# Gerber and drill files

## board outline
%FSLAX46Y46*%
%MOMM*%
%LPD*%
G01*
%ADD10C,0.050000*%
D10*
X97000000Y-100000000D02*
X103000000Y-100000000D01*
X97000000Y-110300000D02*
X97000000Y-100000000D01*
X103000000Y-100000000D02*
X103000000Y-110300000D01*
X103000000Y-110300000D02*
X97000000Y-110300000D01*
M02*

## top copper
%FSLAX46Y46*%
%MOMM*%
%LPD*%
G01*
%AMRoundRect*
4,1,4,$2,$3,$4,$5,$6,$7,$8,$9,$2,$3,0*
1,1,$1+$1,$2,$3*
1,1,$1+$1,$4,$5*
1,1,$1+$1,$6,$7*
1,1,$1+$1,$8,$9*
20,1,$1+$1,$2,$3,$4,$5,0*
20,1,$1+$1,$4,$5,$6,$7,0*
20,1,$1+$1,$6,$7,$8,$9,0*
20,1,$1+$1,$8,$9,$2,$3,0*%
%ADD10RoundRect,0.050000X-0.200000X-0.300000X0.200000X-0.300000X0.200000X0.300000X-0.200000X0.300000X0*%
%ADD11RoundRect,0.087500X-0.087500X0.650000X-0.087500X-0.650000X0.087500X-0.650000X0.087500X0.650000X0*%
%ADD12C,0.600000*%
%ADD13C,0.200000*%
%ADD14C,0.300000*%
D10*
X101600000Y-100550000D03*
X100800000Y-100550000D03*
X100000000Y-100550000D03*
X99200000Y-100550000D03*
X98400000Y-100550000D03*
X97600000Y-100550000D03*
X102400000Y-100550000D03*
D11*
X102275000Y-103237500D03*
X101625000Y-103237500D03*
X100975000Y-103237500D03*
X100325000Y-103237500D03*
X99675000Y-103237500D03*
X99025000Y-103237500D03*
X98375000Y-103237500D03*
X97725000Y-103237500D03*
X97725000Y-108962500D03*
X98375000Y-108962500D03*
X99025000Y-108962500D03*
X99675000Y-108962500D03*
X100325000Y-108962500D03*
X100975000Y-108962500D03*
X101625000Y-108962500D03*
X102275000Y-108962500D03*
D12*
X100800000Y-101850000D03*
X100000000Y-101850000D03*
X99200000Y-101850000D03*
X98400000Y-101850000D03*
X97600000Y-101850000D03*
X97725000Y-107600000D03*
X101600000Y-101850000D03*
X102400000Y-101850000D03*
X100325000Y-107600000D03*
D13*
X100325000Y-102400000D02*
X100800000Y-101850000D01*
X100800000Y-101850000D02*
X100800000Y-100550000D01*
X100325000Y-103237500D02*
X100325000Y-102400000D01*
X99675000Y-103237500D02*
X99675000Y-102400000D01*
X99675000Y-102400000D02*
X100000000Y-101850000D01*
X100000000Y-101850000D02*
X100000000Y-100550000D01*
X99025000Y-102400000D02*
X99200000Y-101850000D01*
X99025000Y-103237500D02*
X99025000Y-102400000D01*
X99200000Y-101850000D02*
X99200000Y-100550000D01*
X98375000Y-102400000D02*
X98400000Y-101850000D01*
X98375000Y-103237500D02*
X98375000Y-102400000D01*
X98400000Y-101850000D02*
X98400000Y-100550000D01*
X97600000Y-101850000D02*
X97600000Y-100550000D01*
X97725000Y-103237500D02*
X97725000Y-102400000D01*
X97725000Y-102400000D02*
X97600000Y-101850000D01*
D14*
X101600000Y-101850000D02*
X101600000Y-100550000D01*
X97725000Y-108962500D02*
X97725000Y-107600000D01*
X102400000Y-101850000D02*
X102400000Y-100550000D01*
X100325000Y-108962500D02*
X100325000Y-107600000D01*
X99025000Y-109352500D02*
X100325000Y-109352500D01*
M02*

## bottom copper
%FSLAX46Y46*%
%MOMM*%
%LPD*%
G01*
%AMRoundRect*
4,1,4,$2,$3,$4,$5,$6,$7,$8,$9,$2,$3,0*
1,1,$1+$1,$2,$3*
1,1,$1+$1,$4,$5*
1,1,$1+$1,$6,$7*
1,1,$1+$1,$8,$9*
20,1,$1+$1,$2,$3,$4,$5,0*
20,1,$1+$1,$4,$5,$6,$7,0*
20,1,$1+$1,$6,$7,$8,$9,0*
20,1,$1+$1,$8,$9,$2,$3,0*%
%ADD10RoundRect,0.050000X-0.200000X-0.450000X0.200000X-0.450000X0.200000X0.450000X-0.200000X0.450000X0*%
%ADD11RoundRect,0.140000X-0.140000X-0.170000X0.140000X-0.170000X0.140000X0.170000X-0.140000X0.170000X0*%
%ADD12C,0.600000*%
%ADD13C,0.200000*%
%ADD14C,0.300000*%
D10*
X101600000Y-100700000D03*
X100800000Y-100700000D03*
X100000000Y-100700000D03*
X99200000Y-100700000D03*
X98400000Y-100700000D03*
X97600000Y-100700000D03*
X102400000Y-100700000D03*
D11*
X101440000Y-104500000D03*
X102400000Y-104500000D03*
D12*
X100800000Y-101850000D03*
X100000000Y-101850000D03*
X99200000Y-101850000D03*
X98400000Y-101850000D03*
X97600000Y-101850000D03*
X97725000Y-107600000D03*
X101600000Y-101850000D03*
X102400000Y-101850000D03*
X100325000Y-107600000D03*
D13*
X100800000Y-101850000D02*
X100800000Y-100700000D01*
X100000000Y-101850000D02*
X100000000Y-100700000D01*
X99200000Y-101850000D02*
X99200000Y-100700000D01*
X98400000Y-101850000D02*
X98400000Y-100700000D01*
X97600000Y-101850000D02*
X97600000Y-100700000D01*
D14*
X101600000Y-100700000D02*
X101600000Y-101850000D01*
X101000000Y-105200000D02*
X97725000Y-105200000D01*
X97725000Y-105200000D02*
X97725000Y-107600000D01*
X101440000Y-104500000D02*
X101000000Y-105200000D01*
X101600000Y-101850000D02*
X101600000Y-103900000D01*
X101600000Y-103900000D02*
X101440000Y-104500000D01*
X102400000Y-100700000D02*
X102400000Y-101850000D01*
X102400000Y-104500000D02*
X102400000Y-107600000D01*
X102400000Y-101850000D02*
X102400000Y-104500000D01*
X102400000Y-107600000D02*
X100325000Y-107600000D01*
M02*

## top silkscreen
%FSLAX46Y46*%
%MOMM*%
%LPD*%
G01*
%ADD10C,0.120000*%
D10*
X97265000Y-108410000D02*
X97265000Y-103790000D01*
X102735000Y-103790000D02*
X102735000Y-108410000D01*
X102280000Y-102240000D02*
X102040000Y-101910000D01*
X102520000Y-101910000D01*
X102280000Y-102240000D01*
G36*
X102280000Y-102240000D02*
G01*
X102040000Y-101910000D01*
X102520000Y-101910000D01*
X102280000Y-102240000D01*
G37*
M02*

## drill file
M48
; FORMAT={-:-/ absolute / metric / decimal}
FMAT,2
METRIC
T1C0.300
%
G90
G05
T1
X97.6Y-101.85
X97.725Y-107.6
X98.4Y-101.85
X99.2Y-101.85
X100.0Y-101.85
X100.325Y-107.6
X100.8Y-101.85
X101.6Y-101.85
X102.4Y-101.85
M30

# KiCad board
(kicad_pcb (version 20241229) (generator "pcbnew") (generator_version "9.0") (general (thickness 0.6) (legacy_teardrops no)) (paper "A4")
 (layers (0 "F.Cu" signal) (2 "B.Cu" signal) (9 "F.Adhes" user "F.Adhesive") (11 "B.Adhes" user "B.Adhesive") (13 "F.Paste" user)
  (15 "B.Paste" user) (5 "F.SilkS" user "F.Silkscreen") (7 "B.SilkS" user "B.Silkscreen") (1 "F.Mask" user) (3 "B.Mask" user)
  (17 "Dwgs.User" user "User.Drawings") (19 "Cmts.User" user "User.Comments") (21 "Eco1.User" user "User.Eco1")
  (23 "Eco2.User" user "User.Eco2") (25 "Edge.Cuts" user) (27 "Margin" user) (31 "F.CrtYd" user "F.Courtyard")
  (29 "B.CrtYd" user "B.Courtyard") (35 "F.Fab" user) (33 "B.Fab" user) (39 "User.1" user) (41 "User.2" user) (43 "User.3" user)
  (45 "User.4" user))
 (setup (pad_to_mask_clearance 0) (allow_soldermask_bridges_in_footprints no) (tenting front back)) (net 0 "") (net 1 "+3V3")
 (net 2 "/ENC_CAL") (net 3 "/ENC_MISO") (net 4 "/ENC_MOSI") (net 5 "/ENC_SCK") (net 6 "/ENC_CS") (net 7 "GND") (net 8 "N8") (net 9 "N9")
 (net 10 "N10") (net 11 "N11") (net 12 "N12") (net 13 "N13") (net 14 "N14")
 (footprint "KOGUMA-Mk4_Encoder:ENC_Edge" (layer "F.Cu") (at 100 100)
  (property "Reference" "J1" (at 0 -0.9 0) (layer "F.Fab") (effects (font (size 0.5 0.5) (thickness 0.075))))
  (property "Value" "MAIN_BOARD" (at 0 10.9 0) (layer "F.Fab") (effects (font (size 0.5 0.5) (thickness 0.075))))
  (pad "1" smd roundrect (at 1.6 0.55) (size 0.5 0.7) (layers "F.Cu" "F.Mask" "F.Paste") (roundrect_rratio 0.1) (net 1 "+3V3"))
  (pad "1" smd roundrect (at 1.6 0.7) (size 0.5 1) (layers "B.Cu" "B.Mask" "B.Paste") (roundrect_rratio 0.1) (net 1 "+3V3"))
  (pad "2" smd roundrect (at 0.8 0.55) (size 0.5 0.7) (layers "F.Cu" "F.Mask" "F.Paste") (roundrect_rratio 0.1) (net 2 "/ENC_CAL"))
  (pad "2" smd roundrect (at 0.8 0.7) (size 0.5 1) (layers "B.Cu" "B.Mask" "B.Paste") (roundrect_rratio 0.1) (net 2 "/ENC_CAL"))
  (pad "3" smd roundrect (at 0 0.55) (size 0.5 0.7) (layers "F.Cu" "F.Mask" "F.Paste") (roundrect_rratio 0.1) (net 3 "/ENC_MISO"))
  (pad "3" smd roundrect (at 0 0.7) (size 0.5 1) (layers "B.Cu" "B.Mask" "B.Paste") (roundrect_rratio 0.1) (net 3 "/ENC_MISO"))
  (pad "4" smd roundrect (at -0.8 0.55) (size 0.5 0.7) (layers "F.Cu" "F.Mask" "F.Paste") (roundrect_rratio 0.1) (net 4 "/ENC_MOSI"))
  (pad "4" smd roundrect (at -0.8 0.7) (size 0.5 1) (layers "B.Cu" "B.Mask" "B.Paste") (roundrect_rratio 0.1) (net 4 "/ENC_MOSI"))
  (pad "5" smd roundrect (at -1.6 0.55) (size 0.5 0.7) (layers "F.Cu" "F.Mask" "F.Paste") (roundrect_rratio 0.1) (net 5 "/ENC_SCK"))
  (pad "5" smd roundrect (at -1.6 0.7) (size 0.5 1) (layers "B.Cu" "B.Mask" "B.Paste") (roundrect_rratio 0.1) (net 5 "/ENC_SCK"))
  (pad "6" smd roundrect (at -2.4 0.55) (size 0.5 0.7) (layers "F.Cu" "F.Mask" "F.Paste") (roundrect_rratio 0.1) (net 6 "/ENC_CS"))
  (pad "6" smd roundrect (at -2.4 0.7) (size 0.5 1) (layers "B.Cu" "B.Mask" "B.Paste") (roundrect_rratio 0.1) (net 6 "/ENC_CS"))
  (pad "7" smd roundrect (at 2.4 0.55) (size 0.5 0.7) (layers "F.Cu" "F.Mask" "F.Paste") (roundrect_rratio 0.1) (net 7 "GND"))
  (pad "7" smd roundrect (at 2.4 0.7) (size 0.5 1) (layers "B.Cu" "B.Mask" "B.Paste") (roundrect_rratio 0.1) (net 7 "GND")))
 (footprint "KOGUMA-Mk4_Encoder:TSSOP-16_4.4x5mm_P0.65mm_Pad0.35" (layer "F.Cu") (at 100 106.1 -90)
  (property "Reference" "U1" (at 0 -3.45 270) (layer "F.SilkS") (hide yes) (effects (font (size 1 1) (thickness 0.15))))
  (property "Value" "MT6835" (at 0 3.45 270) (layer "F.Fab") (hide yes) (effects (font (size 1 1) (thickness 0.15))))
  (fp_line (start 2.31 2.735) (end -2.31 2.735) (stroke (width 0.12) (type solid)) (layer "F.SilkS"))
  (fp_line (start -2.31 -2.735) (end 2.31 -2.735) (stroke (width 0.12) (type solid)) (layer "F.SilkS"))
  (fp_poly (pts (xy -3.86 -2.28) (xy -4.19 -2.04) (xy -4.19 -2.52)) (stroke (width 0.12) (type solid)) (fill yes) (layer "F.SilkS"))
  (pad "1" smd roundrect (at -2.8625 -2.275 270) (size 1.475 0.35) (layers "F.Cu" "F.Mask" "F.Paste") (roundrect_rratio 0.25) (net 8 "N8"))
  (pad "2" smd roundrect (at -2.8625 -1.625 270) (size 1.475 0.35) (layers "F.Cu" "F.Mask" "F.Paste") (roundrect_rratio 0.25) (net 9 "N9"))
  (pad "3" smd roundrect (at -2.8625 -0.975 270) (size 1.475 0.35) (layers "F.Cu" "F.Mask" "F.Paste") (roundrect_rratio 0.25) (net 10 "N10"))
  (pad "4" smd roundrect (at -2.8625 -0.325 270) (size 1.475 0.35) (layers "F.Cu" "F.Mask" "F.Paste") (roundrect_rratio 0.25)
   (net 2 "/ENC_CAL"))
  (pad "5" smd roundrect (at -2.8625 0.325 270) (size 1.475 0.35) (layers "F.Cu" "F.Mask" "F.Paste") (roundrect_rratio 0.25)
   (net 3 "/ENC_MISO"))
  (pad "6" smd roundrect (at -2.8625 0.975 270) (size 1.475 0.35) (layers "F.Cu" "F.Mask" "F.Paste") (roundrect_rratio 0.25)
   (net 4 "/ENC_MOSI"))
  (pad "7" smd roundrect (at -2.8625 1.625 270) (size 1.475 0.35) (layers "F.Cu" "F.Mask" "F.Paste") (roundrect_rratio 0.25)
   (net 5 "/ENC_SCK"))
  (pad "8" smd roundrect (at -2.8625 2.275 270) (size 1.475 0.35) (layers "F.Cu" "F.Mask" "F.Paste") (roundrect_rratio 0.25)
   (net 6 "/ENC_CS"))
  (pad "9" smd roundrect (at 2.8625 2.275 270) (size 1.475 0.35) (layers "F.Cu" "F.Mask" "F.Paste") (roundrect_rratio 0.25) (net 1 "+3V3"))
  (pad "10" smd roundrect (at 2.8625 1.625 270) (size 1.475 0.35) (layers "F.Cu" "F.Mask" "F.Paste") (roundrect_rratio 0.25) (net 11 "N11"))
  (pad "11" smd roundrect (at 2.8625 0.975 270) (size 1.475 0.35) (layers "F.Cu" "F.Mask" "F.Paste") (roundrect_rratio 0.25) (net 7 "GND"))
  (pad "12" smd roundrect (at 2.8625 0.325 270) (size 1.475 0.35) (layers "F.Cu" "F.Mask" "F.Paste") (roundrect_rratio 0.25) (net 7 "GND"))
  (pad "13" smd roundrect (at 2.8625 -0.325 270) (size 1.475 0.35) (layers "F.Cu" "F.Mask" "F.Paste") (roundrect_rratio 0.25) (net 7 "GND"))
  (pad "14" smd roundrect (at 2.8625 -0.975 270) (size 1.475 0.35) (layers "F.Cu" "F.Mask" "F.Paste") (roundrect_rratio 0.25) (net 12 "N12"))
  (pad "15" smd roundrect (at 2.8625 -1.625 270) (size 1.475 0.35) (layers "F.Cu" "F.Mask" "F.Paste") (roundrect_rratio 0.25) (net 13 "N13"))
  (pad "16" smd roundrect (at 2.8625 -2.275 270) (size 1.475 0.35) (layers "F.Cu" "F.Mask" "F.Paste") (roundrect_rratio 0.25) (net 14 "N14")))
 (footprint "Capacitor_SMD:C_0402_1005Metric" (layer "B.Cu") (at 101.92 104.5)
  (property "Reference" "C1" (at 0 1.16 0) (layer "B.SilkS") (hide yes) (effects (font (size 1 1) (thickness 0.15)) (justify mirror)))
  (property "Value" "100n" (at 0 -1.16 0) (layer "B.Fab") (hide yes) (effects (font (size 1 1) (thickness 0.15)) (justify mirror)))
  (pad "1" smd roundrect (at -0.48 0) (size 0.56 0.62) (layers "B.Cu" "B.Mask" "B.Paste") (roundrect_rratio 0.25) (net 1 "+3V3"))
  (pad "2" smd roundrect (at 0.48 0) (size 0.56 0.62) (layers "B.Cu" "B.Mask" "B.Paste") (roundrect_rratio 0.25) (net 7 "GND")))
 (gr_line (start 97 100) (end 103 100) (stroke (width 0.05) (type default)) (layer "Edge.Cuts"))
 (gr_line (start 97 110.3) (end 97 100) (stroke (width 0.05) (type default)) (layer "Edge.Cuts"))
 (gr_line (start 103 100) (end 103 110.3) (stroke (width 0.05) (type default)) (layer "Edge.Cuts"))
 (gr_line (start 103 110.3) (end 97 110.3) (stroke (width 0.05) (type default)) (layer "Edge.Cuts"))
 (segment (start 100.325 102.4) (end 100.8 101.85) (width 0.2) (layer "F.Cu") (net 2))
 (segment (start 100.8 101.85) (end 100.8 100.55) (width 0.2) (layer "F.Cu") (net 2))
 (segment (start 100.325 103.2375) (end 100.325 102.4) (width 0.2) (layer "F.Cu") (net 2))
 (via (at 100.8 101.85) (size 0.6) (drill 0.3) (layers "F.Cu" "B.Cu") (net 2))
 (segment (start 100.8 101.85) (end 100.8 100.7) (width 0.2) (layer "B.Cu") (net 2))
 (segment (start 99.675 103.2375) (end 99.675 102.4) (width 0.2) (layer "F.Cu") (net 3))
 (segment (start 99.675 102.4) (end 100 101.85) (width 0.2) (layer "F.Cu") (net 3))
 (segment (start 100 101.85) (end 100 100.55) (width 0.2) (layer "F.Cu") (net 3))
 (via (at 100 101.85) (size 0.6) (drill 0.3) (layers "F.Cu" "B.Cu") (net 3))
 (segment (start 100 101.85) (end 100 100.7) (width 0.2) (layer "B.Cu") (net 3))
 (segment (start 99.025 102.4) (end 99.2 101.85) (width 0.2) (layer "F.Cu") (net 4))
 (segment (start 99.025 103.2375) (end 99.025 102.4) (width 0.2) (layer "F.Cu") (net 4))
 (segment (start 99.2 101.85) (end 99.2 100.55) (width 0.2) (layer "F.Cu") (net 4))
 (via (at 99.2 101.85) (size 0.6) (drill 0.3) (layers "F.Cu" "B.Cu") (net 4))
 (segment (start 99.2 101.85) (end 99.2 100.7) (width 0.2) (layer "B.Cu") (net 4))
 (segment (start 98.375 102.4) (end 98.4 101.85) (width 0.2) (layer "F.Cu") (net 5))
 (segment (start 98.375 103.2375) (end 98.375 102.4) (width 0.2) (layer "F.Cu") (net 5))
 (segment (start 98.4 101.85) (end 98.4 100.55) (width 0.2) (layer "F.Cu") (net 5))
 (via (at 98.4 101.85) (size 0.6) (drill 0.3) (layers "F.Cu" "B.Cu") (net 5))
 (segment (start 98.4 101.85) (end 98.4 100.7) (width 0.2) (layer "B.Cu") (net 5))
 (segment (start 97.6 101.85) (end 97.6 100.55) (width 0.2) (layer "F.Cu") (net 6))
 (segment (start 97.725 103.2375) (end 97.725 102.4) (width 0.2) (layer "F.Cu") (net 6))
 (segment (start 97.725 102.4) (end 97.6 101.85) (width 0.2) (layer "F.Cu") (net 6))
 (via (at 97.6 101.85) (size 0.6) (drill 0.3) (layers "F.Cu" "B.Cu") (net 6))
 (segment (start 97.6 101.85) (end 97.6 100.7) (width 0.2) (layer "B.Cu") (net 6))
 (segment (start 101.6 101.85) (end 101.6 100.55) (width 0.3) (layer "F.Cu") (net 1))
 (segment (start 97.725 108.9625) (end 97.725 107.6) (width 0.3) (layer "F.Cu") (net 1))
 (via (at 97.725 107.6) (size 0.6) (drill 0.3) (layers "F.Cu" "B.Cu") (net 1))
 (via (at 101.6 101.85) (size 0.6) (drill 0.3) (layers "F.Cu" "B.Cu") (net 1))
 (segment (start 101.6 100.7) (end 101.6 101.85) (width 0.3) (layer "B.Cu") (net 1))
 (segment (start 101 105.2) (end 97.725 105.2) (width 0.3) (layer "B.Cu") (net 1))
 (segment (start 97.725 105.2) (end 97.725 107.6) (width 0.3) (layer "B.Cu") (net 1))
 (segment (start 101.44 104.5) (end 101 105.2) (width 0.3) (layer "B.Cu") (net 1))
 (segment (start 101.6 101.85) (end 101.6 103.9) (width 0.3) (layer "B.Cu") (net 1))
 (segment (start 101.6 103.9) (end 101.44 104.5) (width 0.3) (layer "B.Cu") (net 1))
 (segment (start 102.4 101.85) (end 102.4 100.55) (width 0.3) (layer "F.Cu") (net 7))
 (segment (start 100.325 108.9625) (end 100.325 107.6) (width 0.3) (layer "F.Cu") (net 7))
 (segment (start 99.025 109.3525) (end 100.325 109.3525) (width 0.3) (layer "F.Cu") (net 7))
 (via (at 102.4 101.85) (size 0.6) (drill 0.3) (layers "F.Cu" "B.Cu") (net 7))
 (via (at 100.325 107.6) (size 0.6) (drill 0.3) (layers "F.Cu" "B.Cu") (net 7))
 (segment (start 102.4 100.7) (end 102.4 101.85) (width 0.3) (layer "B.Cu") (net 7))
 (segment (start 102.4 104.5) (end 102.4 107.6) (width 0.3) (layer "B.Cu") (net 7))
 (segment (start 102.4 101.85) (end 102.4 104.5) (width 0.3) (layer "B.Cu") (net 7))
 (segment (start 102.4 107.6) (end 100.325 107.6) (width 0.3) (layer "B.Cu") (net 7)))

